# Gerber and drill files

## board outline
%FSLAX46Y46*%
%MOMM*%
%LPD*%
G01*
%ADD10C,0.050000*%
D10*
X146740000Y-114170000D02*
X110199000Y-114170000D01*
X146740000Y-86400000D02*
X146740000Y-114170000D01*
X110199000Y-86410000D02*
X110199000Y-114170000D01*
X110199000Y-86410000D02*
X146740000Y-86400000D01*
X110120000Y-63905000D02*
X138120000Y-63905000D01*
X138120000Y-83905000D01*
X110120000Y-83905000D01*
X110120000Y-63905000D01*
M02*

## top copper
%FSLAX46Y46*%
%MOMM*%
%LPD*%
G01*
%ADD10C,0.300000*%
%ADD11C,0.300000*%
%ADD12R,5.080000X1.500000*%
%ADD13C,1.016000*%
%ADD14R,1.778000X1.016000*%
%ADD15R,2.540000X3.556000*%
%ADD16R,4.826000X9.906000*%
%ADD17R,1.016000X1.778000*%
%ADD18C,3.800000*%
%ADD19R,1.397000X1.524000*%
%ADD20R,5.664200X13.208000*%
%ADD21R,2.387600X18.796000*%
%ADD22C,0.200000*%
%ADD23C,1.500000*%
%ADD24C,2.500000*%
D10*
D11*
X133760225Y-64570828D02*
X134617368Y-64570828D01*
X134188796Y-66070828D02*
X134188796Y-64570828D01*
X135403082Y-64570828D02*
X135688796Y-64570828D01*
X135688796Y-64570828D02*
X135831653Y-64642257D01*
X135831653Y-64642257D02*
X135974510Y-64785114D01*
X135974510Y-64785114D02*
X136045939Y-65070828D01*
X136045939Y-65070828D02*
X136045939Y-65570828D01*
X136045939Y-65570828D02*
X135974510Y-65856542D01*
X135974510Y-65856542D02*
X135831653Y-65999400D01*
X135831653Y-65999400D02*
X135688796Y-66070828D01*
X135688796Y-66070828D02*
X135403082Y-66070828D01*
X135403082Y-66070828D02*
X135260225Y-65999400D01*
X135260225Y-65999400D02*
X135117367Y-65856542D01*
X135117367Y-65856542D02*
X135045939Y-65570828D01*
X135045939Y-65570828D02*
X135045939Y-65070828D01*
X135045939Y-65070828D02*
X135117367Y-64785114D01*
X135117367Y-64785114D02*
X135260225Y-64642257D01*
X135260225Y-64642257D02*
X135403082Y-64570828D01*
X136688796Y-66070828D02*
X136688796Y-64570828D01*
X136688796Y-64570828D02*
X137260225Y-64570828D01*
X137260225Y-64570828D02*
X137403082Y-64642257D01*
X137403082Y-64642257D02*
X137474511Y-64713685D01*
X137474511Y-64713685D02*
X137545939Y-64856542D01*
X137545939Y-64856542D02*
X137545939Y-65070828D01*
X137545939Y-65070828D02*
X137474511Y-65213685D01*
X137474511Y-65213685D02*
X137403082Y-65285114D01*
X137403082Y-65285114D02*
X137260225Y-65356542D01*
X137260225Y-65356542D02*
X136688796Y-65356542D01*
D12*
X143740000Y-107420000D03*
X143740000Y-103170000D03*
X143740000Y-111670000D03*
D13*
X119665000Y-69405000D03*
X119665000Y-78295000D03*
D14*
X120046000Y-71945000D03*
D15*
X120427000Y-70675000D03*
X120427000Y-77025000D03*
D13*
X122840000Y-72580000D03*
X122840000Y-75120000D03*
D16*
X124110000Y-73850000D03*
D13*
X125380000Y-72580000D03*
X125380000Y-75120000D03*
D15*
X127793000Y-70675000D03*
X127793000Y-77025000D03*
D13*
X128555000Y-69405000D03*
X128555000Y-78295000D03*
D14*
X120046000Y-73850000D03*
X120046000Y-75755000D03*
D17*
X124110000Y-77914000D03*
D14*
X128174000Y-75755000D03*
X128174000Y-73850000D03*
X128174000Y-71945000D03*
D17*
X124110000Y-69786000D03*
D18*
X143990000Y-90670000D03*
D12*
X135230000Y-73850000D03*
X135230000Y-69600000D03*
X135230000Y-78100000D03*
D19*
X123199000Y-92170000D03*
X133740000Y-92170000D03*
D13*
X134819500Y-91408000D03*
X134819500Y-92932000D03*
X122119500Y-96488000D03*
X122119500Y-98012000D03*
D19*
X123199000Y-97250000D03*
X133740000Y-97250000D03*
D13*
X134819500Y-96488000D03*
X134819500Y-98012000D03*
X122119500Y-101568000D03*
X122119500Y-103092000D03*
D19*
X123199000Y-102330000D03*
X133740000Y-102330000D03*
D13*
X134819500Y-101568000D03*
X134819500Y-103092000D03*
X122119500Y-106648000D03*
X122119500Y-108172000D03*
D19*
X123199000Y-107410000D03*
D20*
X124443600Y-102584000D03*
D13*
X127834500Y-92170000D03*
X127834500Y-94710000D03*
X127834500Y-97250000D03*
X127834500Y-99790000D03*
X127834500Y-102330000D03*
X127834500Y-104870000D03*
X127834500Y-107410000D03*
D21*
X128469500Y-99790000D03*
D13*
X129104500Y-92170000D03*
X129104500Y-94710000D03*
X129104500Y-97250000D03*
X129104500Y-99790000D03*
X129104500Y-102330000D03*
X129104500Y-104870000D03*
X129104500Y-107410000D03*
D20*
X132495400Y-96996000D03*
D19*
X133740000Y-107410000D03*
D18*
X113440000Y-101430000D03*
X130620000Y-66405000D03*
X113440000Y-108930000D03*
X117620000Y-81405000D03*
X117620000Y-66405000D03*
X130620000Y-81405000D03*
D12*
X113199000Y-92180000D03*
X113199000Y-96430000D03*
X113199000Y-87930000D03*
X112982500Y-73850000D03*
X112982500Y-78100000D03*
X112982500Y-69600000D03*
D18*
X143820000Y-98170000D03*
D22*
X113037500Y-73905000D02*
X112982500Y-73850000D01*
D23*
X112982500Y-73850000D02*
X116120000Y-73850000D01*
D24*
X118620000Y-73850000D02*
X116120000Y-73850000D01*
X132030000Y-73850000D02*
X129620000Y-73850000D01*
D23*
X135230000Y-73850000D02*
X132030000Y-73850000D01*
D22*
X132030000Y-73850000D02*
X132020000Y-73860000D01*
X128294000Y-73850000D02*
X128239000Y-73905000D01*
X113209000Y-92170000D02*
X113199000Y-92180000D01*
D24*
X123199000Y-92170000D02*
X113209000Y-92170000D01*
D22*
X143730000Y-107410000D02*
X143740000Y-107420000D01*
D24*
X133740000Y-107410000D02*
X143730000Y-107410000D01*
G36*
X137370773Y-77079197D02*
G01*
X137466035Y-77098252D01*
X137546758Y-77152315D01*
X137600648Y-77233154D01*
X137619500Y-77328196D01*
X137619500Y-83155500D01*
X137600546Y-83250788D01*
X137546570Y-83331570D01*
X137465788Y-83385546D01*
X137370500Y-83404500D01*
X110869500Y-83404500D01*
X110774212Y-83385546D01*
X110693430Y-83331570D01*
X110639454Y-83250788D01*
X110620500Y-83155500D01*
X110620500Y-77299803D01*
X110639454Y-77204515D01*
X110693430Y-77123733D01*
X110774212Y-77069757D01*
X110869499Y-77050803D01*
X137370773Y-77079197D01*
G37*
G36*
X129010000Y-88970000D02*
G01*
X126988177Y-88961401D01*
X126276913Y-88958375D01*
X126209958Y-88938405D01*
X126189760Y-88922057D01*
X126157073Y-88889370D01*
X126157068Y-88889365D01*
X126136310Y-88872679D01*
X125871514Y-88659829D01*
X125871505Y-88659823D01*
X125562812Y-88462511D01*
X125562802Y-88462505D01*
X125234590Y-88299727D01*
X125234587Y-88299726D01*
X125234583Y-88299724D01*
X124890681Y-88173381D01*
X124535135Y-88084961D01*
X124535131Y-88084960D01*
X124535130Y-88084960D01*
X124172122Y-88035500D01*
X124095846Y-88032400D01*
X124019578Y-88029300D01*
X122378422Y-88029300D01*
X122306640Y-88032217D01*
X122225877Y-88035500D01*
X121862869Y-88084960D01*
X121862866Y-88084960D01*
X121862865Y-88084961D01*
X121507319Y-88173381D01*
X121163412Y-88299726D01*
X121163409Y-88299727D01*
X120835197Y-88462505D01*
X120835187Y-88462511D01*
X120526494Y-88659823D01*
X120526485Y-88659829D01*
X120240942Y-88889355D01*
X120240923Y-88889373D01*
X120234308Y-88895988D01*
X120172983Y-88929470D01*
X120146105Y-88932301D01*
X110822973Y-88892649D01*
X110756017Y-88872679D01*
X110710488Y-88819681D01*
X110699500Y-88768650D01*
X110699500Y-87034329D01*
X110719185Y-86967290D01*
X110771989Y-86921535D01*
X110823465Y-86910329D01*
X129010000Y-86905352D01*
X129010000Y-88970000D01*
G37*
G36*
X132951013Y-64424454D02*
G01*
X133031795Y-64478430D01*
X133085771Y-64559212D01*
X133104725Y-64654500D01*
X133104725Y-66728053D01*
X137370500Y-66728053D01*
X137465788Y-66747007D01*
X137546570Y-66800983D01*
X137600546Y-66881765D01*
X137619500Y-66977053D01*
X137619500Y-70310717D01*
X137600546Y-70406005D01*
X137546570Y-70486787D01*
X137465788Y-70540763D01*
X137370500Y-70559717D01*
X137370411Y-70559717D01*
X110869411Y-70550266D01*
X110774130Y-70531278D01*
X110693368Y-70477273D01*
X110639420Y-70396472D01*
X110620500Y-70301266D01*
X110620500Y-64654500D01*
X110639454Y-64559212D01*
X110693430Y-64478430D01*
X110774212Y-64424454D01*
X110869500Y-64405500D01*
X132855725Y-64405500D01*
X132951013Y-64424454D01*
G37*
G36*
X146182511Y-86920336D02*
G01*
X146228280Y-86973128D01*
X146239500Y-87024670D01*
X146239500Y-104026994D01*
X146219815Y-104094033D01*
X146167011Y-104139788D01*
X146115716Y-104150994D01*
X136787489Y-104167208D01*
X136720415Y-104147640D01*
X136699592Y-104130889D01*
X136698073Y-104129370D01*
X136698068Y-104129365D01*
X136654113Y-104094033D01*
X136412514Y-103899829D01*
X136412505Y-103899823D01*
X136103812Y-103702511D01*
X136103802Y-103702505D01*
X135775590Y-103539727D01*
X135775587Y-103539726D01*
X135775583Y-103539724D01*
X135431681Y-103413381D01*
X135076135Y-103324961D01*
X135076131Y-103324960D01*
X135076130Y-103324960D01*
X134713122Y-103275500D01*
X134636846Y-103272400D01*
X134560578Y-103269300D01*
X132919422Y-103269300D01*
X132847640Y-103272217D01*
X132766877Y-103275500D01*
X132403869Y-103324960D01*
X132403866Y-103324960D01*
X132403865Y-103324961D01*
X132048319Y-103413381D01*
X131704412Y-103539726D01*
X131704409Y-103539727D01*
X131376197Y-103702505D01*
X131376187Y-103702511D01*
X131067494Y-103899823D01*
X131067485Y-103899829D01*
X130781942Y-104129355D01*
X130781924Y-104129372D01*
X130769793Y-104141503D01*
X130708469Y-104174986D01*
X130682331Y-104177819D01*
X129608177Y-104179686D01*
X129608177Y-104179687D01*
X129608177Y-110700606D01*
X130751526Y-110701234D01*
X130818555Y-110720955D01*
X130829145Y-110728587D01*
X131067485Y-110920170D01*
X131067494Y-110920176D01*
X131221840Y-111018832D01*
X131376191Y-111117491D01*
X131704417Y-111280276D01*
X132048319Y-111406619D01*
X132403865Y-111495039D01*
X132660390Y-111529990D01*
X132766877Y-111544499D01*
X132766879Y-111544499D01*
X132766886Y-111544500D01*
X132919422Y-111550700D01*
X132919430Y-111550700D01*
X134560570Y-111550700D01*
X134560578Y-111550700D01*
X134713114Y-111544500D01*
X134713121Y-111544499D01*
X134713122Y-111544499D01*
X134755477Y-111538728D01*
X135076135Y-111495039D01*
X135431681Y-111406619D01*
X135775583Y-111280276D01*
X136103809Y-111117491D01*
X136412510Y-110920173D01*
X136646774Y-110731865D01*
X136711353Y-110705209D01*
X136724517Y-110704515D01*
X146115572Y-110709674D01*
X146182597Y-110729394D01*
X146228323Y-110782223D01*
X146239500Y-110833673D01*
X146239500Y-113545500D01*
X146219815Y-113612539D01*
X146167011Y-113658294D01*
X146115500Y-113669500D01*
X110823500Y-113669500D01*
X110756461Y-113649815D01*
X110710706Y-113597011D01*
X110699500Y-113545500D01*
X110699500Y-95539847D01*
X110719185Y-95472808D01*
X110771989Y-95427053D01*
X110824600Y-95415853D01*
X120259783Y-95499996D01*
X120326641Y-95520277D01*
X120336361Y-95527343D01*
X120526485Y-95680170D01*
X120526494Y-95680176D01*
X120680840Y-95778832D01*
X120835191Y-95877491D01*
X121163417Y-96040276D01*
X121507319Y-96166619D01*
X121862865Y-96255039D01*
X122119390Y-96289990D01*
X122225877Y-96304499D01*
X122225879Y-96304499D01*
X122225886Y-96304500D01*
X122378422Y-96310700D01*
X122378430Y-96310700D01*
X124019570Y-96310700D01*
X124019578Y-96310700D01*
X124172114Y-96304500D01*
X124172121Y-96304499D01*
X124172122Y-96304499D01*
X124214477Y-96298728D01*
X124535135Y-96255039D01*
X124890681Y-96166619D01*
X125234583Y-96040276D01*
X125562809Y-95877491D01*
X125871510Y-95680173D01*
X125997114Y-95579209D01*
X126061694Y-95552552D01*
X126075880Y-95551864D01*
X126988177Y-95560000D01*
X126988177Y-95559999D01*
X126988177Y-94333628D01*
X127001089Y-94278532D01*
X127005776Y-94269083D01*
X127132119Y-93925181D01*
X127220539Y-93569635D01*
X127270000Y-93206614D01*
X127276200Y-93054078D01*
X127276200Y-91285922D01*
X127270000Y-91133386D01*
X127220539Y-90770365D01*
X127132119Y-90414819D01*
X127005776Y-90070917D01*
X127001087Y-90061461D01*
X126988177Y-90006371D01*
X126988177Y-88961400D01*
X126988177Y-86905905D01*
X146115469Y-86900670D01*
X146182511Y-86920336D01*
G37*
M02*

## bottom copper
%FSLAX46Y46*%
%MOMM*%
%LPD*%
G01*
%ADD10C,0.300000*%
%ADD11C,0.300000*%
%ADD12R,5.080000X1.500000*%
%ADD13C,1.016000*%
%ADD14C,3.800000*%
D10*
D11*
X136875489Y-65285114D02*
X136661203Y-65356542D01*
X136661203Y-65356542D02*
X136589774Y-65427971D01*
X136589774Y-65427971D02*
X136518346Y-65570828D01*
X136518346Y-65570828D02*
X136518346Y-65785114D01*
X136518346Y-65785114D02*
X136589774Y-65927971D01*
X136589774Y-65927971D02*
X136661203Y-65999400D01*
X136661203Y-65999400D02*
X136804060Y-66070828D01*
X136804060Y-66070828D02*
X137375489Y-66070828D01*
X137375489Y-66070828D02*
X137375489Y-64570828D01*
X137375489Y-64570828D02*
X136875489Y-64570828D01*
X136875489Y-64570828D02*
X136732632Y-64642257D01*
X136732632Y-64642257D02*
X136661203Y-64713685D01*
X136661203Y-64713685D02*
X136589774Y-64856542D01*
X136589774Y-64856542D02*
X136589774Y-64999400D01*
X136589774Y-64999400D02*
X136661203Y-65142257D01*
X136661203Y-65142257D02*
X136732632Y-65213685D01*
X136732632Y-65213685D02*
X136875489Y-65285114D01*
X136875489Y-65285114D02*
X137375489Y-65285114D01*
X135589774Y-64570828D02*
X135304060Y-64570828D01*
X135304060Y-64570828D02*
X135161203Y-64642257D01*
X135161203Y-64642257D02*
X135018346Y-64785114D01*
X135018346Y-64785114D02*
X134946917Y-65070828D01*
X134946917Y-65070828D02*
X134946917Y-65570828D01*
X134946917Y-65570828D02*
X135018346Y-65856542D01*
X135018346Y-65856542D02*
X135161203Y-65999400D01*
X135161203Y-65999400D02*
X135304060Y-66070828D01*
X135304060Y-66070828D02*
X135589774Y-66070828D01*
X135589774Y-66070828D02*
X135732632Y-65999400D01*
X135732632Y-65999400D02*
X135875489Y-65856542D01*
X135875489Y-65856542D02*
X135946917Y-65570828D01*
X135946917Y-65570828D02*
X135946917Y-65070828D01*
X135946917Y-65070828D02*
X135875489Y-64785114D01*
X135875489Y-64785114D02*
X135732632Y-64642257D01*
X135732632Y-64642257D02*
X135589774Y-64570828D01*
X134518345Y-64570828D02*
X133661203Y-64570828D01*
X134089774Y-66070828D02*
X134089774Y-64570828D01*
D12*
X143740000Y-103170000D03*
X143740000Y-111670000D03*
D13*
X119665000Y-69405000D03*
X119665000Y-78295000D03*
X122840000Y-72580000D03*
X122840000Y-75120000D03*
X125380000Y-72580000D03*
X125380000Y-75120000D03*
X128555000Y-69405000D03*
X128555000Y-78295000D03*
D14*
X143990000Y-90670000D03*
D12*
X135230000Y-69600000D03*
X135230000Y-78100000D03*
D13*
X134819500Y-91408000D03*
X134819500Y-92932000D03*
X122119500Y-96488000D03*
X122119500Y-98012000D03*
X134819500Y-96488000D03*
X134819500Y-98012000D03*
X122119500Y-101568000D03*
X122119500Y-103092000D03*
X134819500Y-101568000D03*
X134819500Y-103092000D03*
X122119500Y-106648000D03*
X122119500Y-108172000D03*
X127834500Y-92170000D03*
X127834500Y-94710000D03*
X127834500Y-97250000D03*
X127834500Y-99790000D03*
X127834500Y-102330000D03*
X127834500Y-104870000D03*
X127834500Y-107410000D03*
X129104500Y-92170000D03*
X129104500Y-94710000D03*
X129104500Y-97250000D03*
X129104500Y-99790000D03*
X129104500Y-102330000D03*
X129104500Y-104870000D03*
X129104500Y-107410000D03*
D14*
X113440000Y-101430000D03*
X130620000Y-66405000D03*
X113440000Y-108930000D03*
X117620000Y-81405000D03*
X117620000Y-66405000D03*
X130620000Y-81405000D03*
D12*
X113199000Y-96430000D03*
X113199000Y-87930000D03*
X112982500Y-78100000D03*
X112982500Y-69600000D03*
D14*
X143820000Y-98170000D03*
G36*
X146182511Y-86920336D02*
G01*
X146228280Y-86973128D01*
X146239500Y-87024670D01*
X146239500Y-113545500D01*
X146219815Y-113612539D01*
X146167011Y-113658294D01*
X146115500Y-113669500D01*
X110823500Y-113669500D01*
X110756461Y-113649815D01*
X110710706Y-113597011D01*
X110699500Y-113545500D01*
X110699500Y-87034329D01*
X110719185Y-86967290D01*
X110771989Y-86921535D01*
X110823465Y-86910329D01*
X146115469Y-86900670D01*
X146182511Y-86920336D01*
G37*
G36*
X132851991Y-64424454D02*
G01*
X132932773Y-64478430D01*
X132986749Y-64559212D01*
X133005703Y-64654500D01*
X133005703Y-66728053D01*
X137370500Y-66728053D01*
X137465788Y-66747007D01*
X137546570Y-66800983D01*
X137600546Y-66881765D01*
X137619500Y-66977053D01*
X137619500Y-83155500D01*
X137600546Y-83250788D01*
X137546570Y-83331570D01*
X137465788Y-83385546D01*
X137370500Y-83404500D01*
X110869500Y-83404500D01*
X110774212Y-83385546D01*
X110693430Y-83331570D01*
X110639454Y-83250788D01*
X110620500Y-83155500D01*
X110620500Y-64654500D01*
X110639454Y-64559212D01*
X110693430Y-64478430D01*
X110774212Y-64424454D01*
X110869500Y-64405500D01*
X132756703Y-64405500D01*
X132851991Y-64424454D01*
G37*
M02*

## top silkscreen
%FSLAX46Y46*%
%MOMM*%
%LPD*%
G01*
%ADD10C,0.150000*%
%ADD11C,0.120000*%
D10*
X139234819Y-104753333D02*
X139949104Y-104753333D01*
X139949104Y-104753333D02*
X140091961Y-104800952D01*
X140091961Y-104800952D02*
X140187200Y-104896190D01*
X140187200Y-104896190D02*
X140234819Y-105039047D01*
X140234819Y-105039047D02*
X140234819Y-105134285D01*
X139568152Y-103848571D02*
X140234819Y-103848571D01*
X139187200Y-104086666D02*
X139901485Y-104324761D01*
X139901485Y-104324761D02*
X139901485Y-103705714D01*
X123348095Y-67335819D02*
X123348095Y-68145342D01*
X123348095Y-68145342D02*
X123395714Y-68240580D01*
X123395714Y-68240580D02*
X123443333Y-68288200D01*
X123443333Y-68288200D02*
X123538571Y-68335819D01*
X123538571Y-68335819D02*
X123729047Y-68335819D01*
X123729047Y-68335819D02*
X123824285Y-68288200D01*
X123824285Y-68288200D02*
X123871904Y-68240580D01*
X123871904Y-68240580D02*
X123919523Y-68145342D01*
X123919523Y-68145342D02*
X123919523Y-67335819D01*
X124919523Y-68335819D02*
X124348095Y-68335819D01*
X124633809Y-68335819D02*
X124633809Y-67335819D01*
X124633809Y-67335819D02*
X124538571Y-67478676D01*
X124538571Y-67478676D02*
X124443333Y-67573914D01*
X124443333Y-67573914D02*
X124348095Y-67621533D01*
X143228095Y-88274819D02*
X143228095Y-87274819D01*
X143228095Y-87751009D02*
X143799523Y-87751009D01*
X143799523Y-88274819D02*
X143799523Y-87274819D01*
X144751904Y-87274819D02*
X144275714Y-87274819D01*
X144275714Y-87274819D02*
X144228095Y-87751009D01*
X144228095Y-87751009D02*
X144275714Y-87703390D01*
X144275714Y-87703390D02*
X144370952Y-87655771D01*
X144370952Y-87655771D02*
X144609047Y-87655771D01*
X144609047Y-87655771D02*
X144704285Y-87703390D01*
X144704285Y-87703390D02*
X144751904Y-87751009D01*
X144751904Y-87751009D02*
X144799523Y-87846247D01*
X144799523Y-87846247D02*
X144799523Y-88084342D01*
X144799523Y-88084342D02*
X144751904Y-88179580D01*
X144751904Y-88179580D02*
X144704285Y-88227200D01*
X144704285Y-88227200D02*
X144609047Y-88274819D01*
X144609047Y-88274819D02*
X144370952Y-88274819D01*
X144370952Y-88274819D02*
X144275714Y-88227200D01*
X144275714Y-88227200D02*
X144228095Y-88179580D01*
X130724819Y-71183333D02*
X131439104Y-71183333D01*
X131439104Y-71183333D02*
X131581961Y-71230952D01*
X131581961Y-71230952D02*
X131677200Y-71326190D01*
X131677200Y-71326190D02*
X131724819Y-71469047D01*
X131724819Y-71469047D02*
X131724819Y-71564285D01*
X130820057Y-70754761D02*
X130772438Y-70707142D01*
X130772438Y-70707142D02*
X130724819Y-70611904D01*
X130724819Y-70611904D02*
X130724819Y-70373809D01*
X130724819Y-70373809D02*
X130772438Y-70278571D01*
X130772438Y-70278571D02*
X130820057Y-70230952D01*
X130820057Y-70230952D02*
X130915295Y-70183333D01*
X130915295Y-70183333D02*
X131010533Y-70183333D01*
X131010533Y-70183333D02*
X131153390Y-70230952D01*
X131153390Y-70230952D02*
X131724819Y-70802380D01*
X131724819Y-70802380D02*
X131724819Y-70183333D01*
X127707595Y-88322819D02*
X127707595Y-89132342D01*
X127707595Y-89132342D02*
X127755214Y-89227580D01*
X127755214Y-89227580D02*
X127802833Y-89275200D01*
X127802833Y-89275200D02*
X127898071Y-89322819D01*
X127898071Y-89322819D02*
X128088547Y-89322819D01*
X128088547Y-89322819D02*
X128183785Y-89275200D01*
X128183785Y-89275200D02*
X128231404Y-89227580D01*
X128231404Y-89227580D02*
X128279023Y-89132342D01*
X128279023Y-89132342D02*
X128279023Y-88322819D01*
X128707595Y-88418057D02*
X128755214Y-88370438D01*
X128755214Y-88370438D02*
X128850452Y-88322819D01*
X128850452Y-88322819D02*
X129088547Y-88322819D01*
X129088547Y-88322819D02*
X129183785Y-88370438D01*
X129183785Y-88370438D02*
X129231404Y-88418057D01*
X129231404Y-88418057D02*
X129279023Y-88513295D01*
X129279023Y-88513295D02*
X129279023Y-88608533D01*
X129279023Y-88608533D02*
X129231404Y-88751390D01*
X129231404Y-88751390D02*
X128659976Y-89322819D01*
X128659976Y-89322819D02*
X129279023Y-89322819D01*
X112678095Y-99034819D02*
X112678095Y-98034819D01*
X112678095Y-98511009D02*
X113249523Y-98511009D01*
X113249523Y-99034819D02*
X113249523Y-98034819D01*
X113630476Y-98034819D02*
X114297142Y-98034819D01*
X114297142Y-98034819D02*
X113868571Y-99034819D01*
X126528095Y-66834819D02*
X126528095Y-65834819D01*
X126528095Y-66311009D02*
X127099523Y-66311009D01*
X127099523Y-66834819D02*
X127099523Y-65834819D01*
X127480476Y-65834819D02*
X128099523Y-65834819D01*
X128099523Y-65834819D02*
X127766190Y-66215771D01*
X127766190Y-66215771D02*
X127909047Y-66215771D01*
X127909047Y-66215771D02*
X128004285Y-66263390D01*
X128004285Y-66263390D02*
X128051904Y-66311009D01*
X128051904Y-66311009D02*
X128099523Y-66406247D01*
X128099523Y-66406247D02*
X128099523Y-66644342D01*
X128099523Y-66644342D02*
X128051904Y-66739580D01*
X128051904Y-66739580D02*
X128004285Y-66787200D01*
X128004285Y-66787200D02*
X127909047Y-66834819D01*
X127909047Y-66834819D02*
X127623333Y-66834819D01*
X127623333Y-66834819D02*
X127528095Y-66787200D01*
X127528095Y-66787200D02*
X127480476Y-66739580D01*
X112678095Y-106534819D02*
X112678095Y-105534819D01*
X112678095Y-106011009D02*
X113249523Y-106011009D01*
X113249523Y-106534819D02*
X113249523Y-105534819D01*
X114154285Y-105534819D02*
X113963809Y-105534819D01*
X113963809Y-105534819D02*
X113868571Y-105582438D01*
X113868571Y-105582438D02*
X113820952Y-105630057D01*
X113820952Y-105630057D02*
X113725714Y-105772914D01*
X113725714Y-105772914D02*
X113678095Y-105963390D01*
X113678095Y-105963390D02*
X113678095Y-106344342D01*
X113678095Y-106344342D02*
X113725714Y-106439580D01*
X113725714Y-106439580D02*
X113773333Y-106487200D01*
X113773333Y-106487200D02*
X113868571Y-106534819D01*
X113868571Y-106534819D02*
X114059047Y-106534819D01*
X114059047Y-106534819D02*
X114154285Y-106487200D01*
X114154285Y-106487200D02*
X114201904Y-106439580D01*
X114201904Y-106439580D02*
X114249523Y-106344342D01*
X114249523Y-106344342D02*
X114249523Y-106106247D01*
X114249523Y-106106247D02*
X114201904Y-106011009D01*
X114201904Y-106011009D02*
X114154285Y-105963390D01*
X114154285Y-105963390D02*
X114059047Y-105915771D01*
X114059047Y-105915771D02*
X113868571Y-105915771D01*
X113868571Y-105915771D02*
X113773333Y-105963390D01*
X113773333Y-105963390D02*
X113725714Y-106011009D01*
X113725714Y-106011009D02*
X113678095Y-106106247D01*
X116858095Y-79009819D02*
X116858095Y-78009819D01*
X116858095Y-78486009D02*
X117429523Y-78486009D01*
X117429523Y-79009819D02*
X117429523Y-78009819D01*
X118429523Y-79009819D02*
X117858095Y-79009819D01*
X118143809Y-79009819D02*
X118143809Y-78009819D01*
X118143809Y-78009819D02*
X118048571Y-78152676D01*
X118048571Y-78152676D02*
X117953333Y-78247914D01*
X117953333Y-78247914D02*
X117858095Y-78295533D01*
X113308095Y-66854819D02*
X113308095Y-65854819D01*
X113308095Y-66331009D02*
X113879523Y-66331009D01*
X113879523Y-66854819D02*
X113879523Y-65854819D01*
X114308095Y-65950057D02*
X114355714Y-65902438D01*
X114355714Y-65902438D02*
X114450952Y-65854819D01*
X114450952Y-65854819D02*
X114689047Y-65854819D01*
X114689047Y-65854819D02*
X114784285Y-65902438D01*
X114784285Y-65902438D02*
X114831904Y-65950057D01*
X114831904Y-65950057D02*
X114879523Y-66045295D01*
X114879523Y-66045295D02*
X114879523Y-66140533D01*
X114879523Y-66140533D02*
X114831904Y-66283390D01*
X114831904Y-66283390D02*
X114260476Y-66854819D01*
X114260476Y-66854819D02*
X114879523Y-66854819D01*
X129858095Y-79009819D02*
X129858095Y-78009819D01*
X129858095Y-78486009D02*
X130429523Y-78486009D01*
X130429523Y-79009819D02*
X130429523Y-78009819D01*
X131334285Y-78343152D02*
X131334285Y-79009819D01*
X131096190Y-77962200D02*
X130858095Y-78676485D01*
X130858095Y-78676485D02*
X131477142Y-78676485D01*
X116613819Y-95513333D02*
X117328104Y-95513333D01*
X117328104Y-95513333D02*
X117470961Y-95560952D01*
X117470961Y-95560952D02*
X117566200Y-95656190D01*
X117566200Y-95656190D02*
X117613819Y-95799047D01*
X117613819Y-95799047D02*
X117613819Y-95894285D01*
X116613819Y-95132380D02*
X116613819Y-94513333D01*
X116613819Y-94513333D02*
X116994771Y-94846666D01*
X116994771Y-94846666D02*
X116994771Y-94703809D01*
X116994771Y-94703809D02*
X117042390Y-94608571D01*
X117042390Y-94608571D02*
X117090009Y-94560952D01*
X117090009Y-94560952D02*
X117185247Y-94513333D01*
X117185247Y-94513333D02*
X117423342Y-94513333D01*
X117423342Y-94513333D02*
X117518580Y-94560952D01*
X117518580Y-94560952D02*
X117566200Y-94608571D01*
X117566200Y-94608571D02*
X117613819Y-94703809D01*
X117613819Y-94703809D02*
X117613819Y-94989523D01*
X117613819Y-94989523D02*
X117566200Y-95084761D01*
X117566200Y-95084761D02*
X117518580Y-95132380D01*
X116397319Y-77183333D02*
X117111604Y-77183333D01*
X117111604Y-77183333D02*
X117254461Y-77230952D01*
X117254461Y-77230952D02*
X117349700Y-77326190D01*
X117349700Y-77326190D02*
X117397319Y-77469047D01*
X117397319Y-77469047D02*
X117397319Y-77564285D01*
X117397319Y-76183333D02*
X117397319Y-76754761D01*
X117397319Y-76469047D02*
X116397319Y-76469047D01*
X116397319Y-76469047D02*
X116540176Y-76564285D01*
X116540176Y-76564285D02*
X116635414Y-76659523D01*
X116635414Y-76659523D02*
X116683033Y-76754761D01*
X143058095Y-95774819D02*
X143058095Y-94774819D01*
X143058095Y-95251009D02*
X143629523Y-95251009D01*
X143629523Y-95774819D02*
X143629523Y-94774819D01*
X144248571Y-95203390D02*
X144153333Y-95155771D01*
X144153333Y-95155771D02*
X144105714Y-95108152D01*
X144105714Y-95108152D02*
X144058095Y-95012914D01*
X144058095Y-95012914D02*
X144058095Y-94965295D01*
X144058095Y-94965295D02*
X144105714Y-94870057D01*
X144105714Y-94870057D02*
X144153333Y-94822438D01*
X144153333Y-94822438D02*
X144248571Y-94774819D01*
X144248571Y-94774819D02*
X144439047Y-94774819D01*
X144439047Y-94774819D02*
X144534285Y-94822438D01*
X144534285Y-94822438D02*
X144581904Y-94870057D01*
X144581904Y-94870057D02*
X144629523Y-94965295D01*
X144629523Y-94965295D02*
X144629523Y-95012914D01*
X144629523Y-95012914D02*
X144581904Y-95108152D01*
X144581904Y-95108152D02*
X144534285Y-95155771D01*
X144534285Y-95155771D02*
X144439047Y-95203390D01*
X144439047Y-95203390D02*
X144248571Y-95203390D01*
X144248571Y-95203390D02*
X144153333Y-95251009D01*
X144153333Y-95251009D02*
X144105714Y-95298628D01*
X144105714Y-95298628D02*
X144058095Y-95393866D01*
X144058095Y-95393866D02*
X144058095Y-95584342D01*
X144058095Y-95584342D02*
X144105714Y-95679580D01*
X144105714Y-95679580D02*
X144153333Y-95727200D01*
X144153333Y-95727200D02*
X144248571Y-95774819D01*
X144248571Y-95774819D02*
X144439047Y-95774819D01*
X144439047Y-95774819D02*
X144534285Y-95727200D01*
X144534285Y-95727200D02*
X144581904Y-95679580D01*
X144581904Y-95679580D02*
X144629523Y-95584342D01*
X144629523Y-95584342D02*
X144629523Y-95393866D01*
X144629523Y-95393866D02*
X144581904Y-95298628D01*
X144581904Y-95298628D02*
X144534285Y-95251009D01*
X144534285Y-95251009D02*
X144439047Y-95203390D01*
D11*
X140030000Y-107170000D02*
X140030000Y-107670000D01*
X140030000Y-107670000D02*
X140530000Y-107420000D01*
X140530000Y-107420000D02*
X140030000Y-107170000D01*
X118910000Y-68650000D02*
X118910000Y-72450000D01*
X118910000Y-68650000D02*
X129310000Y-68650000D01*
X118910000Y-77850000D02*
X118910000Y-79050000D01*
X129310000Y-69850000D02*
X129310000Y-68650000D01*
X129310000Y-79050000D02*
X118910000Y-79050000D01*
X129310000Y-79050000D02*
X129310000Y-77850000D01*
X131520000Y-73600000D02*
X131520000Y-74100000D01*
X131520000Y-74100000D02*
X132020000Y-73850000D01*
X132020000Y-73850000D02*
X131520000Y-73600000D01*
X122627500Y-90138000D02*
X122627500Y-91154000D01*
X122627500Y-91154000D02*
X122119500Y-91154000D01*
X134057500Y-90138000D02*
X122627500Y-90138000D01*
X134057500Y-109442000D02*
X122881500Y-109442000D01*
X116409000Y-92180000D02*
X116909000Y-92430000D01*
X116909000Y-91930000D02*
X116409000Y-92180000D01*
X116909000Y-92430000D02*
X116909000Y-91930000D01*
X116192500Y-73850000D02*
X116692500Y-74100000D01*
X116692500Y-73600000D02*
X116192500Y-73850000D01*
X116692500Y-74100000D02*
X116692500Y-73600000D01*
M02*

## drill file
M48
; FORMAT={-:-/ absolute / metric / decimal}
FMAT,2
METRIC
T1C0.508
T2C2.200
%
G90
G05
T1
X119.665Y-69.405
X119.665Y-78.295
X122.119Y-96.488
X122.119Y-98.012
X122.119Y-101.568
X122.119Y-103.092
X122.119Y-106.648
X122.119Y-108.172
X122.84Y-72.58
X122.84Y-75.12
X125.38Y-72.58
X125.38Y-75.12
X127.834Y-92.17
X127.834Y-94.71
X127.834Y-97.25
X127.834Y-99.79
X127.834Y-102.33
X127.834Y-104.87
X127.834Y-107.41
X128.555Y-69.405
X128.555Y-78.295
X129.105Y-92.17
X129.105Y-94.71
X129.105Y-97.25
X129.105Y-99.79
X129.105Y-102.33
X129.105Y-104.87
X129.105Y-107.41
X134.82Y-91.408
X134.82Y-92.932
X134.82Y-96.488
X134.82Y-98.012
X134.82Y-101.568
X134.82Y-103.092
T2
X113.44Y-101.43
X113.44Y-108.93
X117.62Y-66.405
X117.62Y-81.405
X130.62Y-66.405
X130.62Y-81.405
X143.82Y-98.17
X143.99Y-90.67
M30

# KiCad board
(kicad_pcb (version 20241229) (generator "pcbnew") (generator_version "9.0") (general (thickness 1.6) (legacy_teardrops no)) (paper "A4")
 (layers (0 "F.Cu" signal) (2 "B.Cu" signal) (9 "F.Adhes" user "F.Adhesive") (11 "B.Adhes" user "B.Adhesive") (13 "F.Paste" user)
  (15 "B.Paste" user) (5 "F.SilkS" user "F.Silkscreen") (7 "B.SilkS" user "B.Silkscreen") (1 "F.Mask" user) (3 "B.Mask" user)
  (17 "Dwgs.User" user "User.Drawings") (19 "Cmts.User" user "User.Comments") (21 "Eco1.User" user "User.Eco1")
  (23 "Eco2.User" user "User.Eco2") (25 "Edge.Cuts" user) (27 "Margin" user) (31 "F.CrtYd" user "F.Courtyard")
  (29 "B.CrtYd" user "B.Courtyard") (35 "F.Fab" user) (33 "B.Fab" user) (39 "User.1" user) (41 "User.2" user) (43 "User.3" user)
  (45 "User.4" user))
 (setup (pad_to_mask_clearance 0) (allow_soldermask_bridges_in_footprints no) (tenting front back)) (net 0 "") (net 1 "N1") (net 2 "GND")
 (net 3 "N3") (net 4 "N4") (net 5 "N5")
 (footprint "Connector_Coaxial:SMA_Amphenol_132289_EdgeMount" (layer "F.Cu") (at 143.74 107.42)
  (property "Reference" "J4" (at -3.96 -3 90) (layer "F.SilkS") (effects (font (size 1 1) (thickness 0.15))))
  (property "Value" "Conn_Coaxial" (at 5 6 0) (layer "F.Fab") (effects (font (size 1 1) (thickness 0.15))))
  (fp_line (start -3.71 -0.25) (end -3.71 0.25) (stroke (width 0.12) (type solid)) (layer "F.SilkS"))
  (fp_line (start -3.71 0.25) (end -3.21 0) (stroke (width 0.12) (type solid)) (layer "F.SilkS"))
  (fp_line (start -3.21 0) (end -3.71 -0.25) (stroke (width 0.12) (type solid)) (layer "F.SilkS"))
  (pad "1" smd rect (at 0 0 90) (size 1.5 5.08) (layers "F.Cu" "F.Mask" "F.Paste") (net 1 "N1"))
  (pad "2" smd rect (at 0 -4.25 90) (size 1.5 5.08) (layers "F.Cu" "F.Mask" "F.Paste") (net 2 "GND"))
  (pad "2" smd rect (at 0 -4.25 90) (size 1.5 5.08) (layers "B.Cu" "B.Mask" "B.Paste") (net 2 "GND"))
  (pad "2" smd rect (at 0 4.25 90) (size 1.5 5.08) (layers "F.Cu" "F.Mask" "F.Paste") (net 2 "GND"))
  (pad "2" smd rect (at 0 4.25 90) (size 1.5 5.08) (layers "B.Cu" "B.Mask" "B.Paste") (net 2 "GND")))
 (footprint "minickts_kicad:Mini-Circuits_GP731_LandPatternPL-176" (layer "F.Cu") (at 124.11 73.85)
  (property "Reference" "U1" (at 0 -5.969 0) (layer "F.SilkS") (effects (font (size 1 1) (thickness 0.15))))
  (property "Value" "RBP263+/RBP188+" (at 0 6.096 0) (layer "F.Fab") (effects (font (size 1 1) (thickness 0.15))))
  (fp_line (start -5.2 -5.2) (end -5.2 -1.4) (stroke (width 0.12) (type solid)) (layer "F.SilkS"))
  (fp_line (start -5.2 -5.2) (end 5.2 -5.2) (stroke (width 0.12) (type solid)) (layer "F.SilkS"))
  (fp_line (start -5.2 4) (end -5.2 5.2) (stroke (width 0.12) (type solid)) (layer "F.SilkS"))
  (fp_line (start 5.2 -4) (end 5.2 -5.2) (stroke (width 0.12) (type solid)) (layer "F.SilkS"))
  (fp_line (start 5.2 5.2) (end -5.2 5.2) (stroke (width 0.12) (type solid)) (layer "F.SilkS"))
  (fp_line (start 5.2 5.2) (end 5.2 4) (stroke (width 0.12) (type solid)) (layer "F.SilkS"))
  (pad "1" thru_hole circle (at -4.445 -4.445) (size 1.016 1.016) (drill 0.508) (layers "*.Cu") (remove_unused_layers no) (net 2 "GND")
   (zone_connect 2))
  (pad "1" thru_hole circle (at -4.445 4.445) (size 1.016 1.016) (drill 0.508) (layers "*.Cu") (remove_unused_layers no) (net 2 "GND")
   (zone_connect 2))
  (pad "1" smd rect (at -4.064 -1.905 180) (size 1.778 1.016) (layers "F.Cu" "F.Mask" "F.Paste") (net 2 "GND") (zone_connect 2))
  (pad "1" smd rect (at -3.683 -3.175) (size 2.54 3.556) (layers "F.Cu") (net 2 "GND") (zone_connect 2))
  (pad "1" smd rect (at -3.683 3.175) (size 2.54 3.556) (layers "F.Cu") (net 2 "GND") (zone_connect 2))
  (pad "1" thru_hole circle (at -1.27 -1.27) (size 1.016 1.016) (drill 0.508) (layers "*.Cu") (remove_unused_layers no) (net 2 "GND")
   (zone_connect 2))
  (pad "1" thru_hole circle (at -1.27 1.27) (size 1.016 1.016) (drill 0.508) (layers "*.Cu") (remove_unused_layers no) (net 2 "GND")
   (zone_connect 2))
  (pad "1" smd rect (at 0 0) (size 4.826 9.906) (layers "F.Cu") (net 2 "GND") (zone_connect 2))
  (pad "1" thru_hole circle (at 1.27 -1.27) (size 1.016 1.016) (drill 0.508) (layers "*.Cu") (remove_unused_layers no) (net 2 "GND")
   (zone_connect 2))
  (pad "1" thru_hole circle (at 1.27 1.27) (size 1.016 1.016) (drill 0.508) (layers "*.Cu") (remove_unused_layers no) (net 2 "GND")
   (zone_connect 2))
  (pad "1" smd rect (at 3.683 -3.175) (size 2.54 3.556) (layers "F.Cu") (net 2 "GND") (zone_connect 2))
  (pad "1" smd rect (at 3.683 3.175) (size 2.54 3.556) (layers "F.Cu") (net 2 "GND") (zone_connect 2))
  (pad "1" thru_hole circle (at 4.445 -4.445) (size 1.016 1.016) (drill 0.508) (layers "*.Cu") (remove_unused_layers no) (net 2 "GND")
   (zone_connect 2))
  (pad "1" thru_hole circle (at 4.445 4.445) (size 1.016 1.016) (drill 0.508) (layers "*.Cu") (remove_unused_layers no) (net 2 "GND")
   (zone_connect 2))
  (pad "2" smd rect (at -4.064 0 180) (size 1.778 1.016) (layers "F.Cu" "F.Mask" "F.Paste") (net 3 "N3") (clearance 0.762))
  (pad "3" smd rect (at -4.064 1.905 180) (size 1.778 1.016) (layers "F.Cu" "F.Mask" "F.Paste") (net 2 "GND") (zone_connect 2))
  (pad "4" smd rect (at 0 4.064 270) (size 1.778 1.016) (layers "F.Cu" "F.Mask" "F.Paste") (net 2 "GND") (zone_connect 2))
  (pad "5" smd rect (at 4.064 1.905) (size 1.778 1.016) (layers "F.Cu" "F.Mask" "F.Paste") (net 2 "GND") (zone_connect 2))
  (pad "6" smd rect (at 4.064 0) (size 1.778 1.016) (layers "F.Cu" "F.Mask" "F.Paste") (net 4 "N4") (clearance 0.762))
  (pad "7" smd rect (at 4.064 -1.905) (size 1.778 1.016) (layers "F.Cu" "F.Mask" "F.Paste") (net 2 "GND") (zone_connect 2))
  (pad "8" smd rect (at 0 -4.064 270) (size 1.778 1.016) (layers "F.Cu" "F.Mask" "F.Paste") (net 2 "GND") (zone_connect 2)))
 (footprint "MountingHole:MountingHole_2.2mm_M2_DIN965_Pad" (layer "F.Cu") (at 143.99 90.67)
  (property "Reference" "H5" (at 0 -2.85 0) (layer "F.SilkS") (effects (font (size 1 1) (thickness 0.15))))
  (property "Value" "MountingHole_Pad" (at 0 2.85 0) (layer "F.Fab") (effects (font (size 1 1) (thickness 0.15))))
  (pad "1" thru_hole circle (at 0 0) (size 3.8 3.8) (drill 2.2) (layers "*.Cu" "*.Mask") (remove_unused_layers no) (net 2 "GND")
   (zone_connect 2)))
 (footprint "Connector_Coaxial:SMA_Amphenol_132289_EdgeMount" (layer "F.Cu") (at 135.23 73.85)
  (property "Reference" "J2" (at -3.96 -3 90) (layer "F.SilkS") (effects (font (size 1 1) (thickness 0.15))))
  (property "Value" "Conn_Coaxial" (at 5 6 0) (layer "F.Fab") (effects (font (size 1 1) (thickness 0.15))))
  (fp_line (start -3.71 -0.25) (end -3.71 0.25) (stroke (width 0.12) (type solid)) (layer "F.SilkS"))
  (fp_line (start -3.71 0.25) (end -3.21 0) (stroke (width 0.12) (type solid)) (layer "F.SilkS"))
  (fp_line (start -3.21 0) (end -3.71 -0.25) (stroke (width 0.12) (type solid)) (layer "F.SilkS"))
  (pad "1" smd rect (at 0 0 90) (size 1.5 5.08) (layers "F.Cu" "F.Mask" "F.Paste") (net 4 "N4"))
  (pad "2" smd rect (at 0 -4.25 90) (size 1.5 5.08) (layers "F.Cu" "F.Mask" "F.Paste") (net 2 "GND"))
  (pad "2" smd rect (at 0 -4.25 90) (size 1.5 5.08) (layers "B.Cu" "B.Mask" "B.Paste") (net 2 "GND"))
  (pad "2" smd rect (at 0 4.25 90) (size 1.5 5.08) (layers "F.Cu" "F.Mask" "F.Paste") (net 2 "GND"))
  (pad "2" smd rect (at 0 4.25 90) (size 1.5 5.08) (layers "B.Cu" "B.Mask" "B.Paste") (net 2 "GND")))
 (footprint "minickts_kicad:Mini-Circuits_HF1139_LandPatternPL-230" (layer "F.Cu") (at 128.4695 99.79)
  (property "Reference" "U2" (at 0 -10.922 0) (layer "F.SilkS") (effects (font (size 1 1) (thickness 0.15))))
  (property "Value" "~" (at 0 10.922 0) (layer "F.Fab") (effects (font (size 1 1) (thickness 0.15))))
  (fp_line (start -5.842 -9.652) (end -5.842 -8.636) (stroke (width 0.12) (type solid)) (layer "F.SilkS"))
  (fp_line (start -5.842 -8.636) (end -6.35 -8.636) (stroke (width 0.12) (type solid)) (layer "F.SilkS"))
  (fp_line (start 5.588 -9.652) (end -5.842 -9.652) (stroke (width 0.12) (type solid)) (layer "F.SilkS"))
  (fp_line (start 5.588 9.652) (end -5.588 9.652) (stroke (width 0.12) (type solid)) (layer "F.SilkS"))
  (pad "1" smd rect (at -5.2705 -7.62 270) (size 1.524 1.397) (layers "F.Cu" "F.Mask" "F.Paste") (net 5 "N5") (clearance 3.3782))
  (pad "2" smd rect (at 5.2705 -7.62 270) (size 1.524 1.397) (layers "F.Cu" "F.Mask" "F.Paste") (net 2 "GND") (zone_connect 2))
  (pad "2" thru_hole circle (at 6.35 -8.382 270) (size 1.016 1.016) (drill 0.508) (layers "*.Cu") (remove_unused_layers no) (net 2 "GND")
   (zone_connect 2))
  (pad "2" thru_hole circle (at 6.35 -6.858 270) (size 1.016 1.016) (drill 0.508) (layers "*.Cu") (remove_unused_layers no) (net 2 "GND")
   (zone_connect 2))
  (pad "3" thru_hole circle (at -6.35 -3.302 270) (size 1.016 1.016) (drill 0.508) (layers "*.Cu") (remove_unused_layers no) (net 2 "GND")
   (zone_connect 2))
  (pad "3" thru_hole circle (at -6.35 -1.778 270) (size 1.016 1.016) (drill 0.508) (layers "*.Cu") (remove_unused_layers no) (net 2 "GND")
   (zone_connect 2))
  (pad "3" smd rect (at -5.2705 -2.54 270) (size 1.524 1.397) (layers "F.Cu" "F.Mask" "F.Paste") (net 2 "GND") (zone_connect 2))
  (pad "4" smd rect (at 5.2705 -2.54 270) (size 1.524 1.397) (layers "F.Cu" "F.Mask" "F.Paste") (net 2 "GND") (zone_connect 2))
  (pad "4" thru_hole circle (at 6.35 -3.302 270) (size 1.016 1.016) (drill 0.508) (layers "*.Cu") (remove_unused_layers no) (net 2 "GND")
   (zone_connect 2))
  (pad "4" thru_hole circle (at 6.35 -1.778 270) (size 1.016 1.016) (drill 0.508) (layers "*.Cu") (remove_unused_layers no) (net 2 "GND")
   (zone_connect 2))
  (pad "5" thru_hole circle (at -6.35 1.778 270) (size 1.016 1.016) (drill 0.508) (layers "*.Cu") (remove_unused_layers no) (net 2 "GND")
   (zone_connect 2))
  (pad "5" thru_hole circle (at -6.35 3.302 270) (size 1.016 1.016) (drill 0.508) (layers "*.Cu") (remove_unused_layers no) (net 2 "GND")
   (zone_connect 2))
  (pad "5" smd rect (at -5.2705 2.54 270) (size 1.524 1.397) (layers "F.Cu" "F.Mask" "F.Paste") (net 2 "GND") (zone_connect 2))
  (pad "6" smd rect (at 5.2705 2.54 270) (size 1.524 1.397) (layers "F.Cu" "F.Mask" "F.Paste") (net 2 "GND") (zone_connect 2))
  (pad "6" thru_hole circle (at 6.35 1.778 270) (size 1.016 1.016) (drill 0.508) (layers "*.Cu") (remove_unused_layers no) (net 2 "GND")
   (zone_connect 2))
  (pad "6" thru_hole circle (at 6.35 3.302 270) (size 1.016 1.016) (drill 0.508) (layers "*.Cu") (remove_unused_layers no) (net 2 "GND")
   (zone_connect 2))
  (pad "7" thru_hole circle (at -6.35 6.858 270) (size 1.016 1.016) (drill 0.508) (layers "*.Cu") (remove_unused_layers no) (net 2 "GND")
   (zone_connect 2))
  (pad "7" thru_hole circle (at -6.35 8.382 270) (size 1.016 1.016) (drill 0.508) (layers "*.Cu") (remove_unused_layers no) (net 2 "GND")
   (zone_connect 2))
  (pad "7" smd rect (at -5.2705 7.62 270) (size 1.524 1.397) (layers "F.Cu" "F.Mask" "F.Paste") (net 2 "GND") (zone_connect 2))
  (pad "7" smd rect (at -4.0259 2.794 270) (size 13.208 5.6642) (layers "F.Cu") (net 2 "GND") (zone_connect 2))
  (pad "7" thru_hole circle (at -0.635 -7.62 270) (size 1.016 1.016) (drill 0.508) (layers "*.Cu") (remove_unused_layers no) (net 2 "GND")
   (zone_connect 2))
  (pad "7" thru_hole circle (at -0.635 -5.08 270) (size 1.016 1.016) (drill 0.508) (layers "*.Cu") (remove_unused_layers no) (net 2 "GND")
   (zone_connect 2))
  (pad "7" thru_hole circle (at -0.635 -2.54 270) (size 1.016 1.016) (drill 0.508) (layers "*.Cu") (remove_unused_layers no) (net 2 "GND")
   (zone_connect 2))
  (pad "7" thru_hole circle (at -0.635 0 270) (size 1.016 1.016) (drill 0.508) (layers "*.Cu") (remove_unused_layers no) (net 2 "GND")
   (zone_connect 2))
  (pad "7" thru_hole circle (at -0.635 2.54 270) (size 1.016 1.016) (drill 0.508) (layers "*.Cu") (remove_unused_layers no) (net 2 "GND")
   (zone_connect 2))
  (pad "7" thru_hole circle (at -0.635 5.08 270) (size 1.016 1.016) (drill 0.508) (layers "*.Cu") (remove_unused_layers no) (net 2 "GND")
   (zone_connect 2))
  (pad "7" thru_hole circle (at -0.635 7.62 270) (size 1.016 1.016) (drill 0.508) (layers "*.Cu") (remove_unused_layers no) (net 2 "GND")
   (zone_connect 2))
  (pad "7" smd rect (at 0 0 270) (size 18.796 2.3876) (layers "F.Cu") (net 2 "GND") (zone_connect 2))
  (pad "7" thru_hole circle (at 0.635 -7.62 270) (size 1.016 1.016) (drill 0.508) (layers "*.Cu") (remove_unused_layers no) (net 2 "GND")
   (zone_connect 2))
  (pad "7" thru_hole circle (at 0.635 -5.08 270) (size 1.016 1.016) (drill 0.508) (layers "*.Cu") (remove_unused_layers no) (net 2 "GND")
   (zone_connect 2))
  (pad "7" thru_hole circle (at 0.635 -2.54 270) (size 1.016 1.016) (drill 0.508) (layers "*.Cu") (remove_unused_layers no) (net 2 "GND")
   (zone_connect 2))
  (pad "7" thru_hole circle (at 0.635 0 270) (size 1.016 1.016) (drill 0.508) (layers "*.Cu") (remove_unused_layers no) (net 2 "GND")
   (zone_connect 2))
  (pad "7" thru_hole circle (at 0.635 2.54 270) (size 1.016 1.016) (drill 0.508) (layers "*.Cu") (remove_unused_layers no) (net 2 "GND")
   (zone_connect 2))
  (pad "7" thru_hole circle (at 0.635 5.08 270) (size 1.016 1.016) (drill 0.508) (layers "*.Cu") (remove_unused_layers no) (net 2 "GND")
   (zone_connect 2))
  (pad "7" thru_hole circle (at 0.635 7.62 270) (size 1.016 1.016) (drill 0.508) (layers "*.Cu") (remove_unused_layers no) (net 2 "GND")
   (zone_connect 2))
  (pad "7" smd rect (at 4.0259 -2.794 270) (size 13.208 5.6642) (layers "F.Cu") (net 2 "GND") (zone_connect 2))
  (pad "8" smd rect (at 5.2705 7.62 270) (size 1.524 1.397) (layers "F.Cu" "F.Mask" "F.Paste") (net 1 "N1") (clearance 3.3782)))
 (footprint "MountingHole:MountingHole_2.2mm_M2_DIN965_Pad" (layer "F.Cu") (at 113.44 101.43)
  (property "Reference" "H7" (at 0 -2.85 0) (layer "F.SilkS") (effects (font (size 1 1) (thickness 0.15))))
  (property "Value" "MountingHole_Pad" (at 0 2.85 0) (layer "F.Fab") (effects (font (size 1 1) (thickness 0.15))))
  (pad "1" thru_hole circle (at 0 0) (size 3.8 3.8) (drill 2.2) (layers "*.Cu" "*.Mask") (remove_unused_layers no) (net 2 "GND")
   (zone_connect 2)))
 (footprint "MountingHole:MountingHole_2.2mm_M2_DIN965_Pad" (layer "F.Cu") (at 130.62 66.405)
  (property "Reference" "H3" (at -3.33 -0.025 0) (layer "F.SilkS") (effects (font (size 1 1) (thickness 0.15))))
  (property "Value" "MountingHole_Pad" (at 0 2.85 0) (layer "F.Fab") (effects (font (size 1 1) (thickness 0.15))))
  (pad "1" thru_hole circle (at 0 0) (size 3.8 3.8) (drill 2.2) (layers "*.Cu" "*.Mask") (remove_unused_layers no) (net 2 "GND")
   (zone_connect 2)))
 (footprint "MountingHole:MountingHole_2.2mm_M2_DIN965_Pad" (layer "F.Cu") (at 113.44 108.93)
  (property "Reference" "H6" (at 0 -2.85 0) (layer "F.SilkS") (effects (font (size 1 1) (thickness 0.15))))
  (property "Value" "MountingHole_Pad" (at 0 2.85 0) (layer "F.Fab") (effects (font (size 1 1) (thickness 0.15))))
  (pad "1" thru_hole circle (at 0 0) (size 3.8 3.8) (drill 2.2) (layers "*.Cu" "*.Mask") (remove_unused_layers no) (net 2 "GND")
   (zone_connect 2)))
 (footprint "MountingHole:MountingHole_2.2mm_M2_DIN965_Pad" (layer "F.Cu") (at 117.62 81.405)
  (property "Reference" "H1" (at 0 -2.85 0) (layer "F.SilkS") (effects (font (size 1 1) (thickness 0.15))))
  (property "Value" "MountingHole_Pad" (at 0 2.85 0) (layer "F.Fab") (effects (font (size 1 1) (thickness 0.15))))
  (pad "1" thru_hole circle (at 0 0) (size 3.8 3.8) (drill 2.2) (layers "*.Cu" "*.Mask") (remove_unused_layers no) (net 2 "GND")
   (zone_connect 2)))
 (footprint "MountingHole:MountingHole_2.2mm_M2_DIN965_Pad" (layer "F.Cu") (at 117.62 66.405)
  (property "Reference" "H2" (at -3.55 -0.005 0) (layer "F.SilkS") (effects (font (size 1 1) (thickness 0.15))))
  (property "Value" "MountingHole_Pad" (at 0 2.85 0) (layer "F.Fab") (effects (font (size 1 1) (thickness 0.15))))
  (pad "1" thru_hole circle (at 0 0) (size 3.8 3.8) (drill 2.2) (layers "*.Cu" "*.Mask") (remove_unused_layers no) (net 2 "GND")
   (zone_connect 2)))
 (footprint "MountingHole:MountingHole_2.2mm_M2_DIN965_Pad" (layer "F.Cu") (at 130.62 81.405)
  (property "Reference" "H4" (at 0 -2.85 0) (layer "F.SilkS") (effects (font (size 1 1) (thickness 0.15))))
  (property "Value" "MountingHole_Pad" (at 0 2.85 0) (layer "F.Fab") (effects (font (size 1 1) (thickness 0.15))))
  (pad "1" thru_hole circle (at 0 0) (size 3.8 3.8) (drill 2.2) (layers "*.Cu" "*.Mask") (remove_unused_layers no) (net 2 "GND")
   (zone_connect 2)))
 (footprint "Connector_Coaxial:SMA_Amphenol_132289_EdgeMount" (layer "F.Cu") (at 113.199 92.18 180)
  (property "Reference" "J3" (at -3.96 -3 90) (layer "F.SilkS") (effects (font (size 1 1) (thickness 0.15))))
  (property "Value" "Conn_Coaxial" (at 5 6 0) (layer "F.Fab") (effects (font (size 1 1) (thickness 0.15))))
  (fp_line (start -3.21 0) (end -3.71 -0.25) (stroke (width 0.12) (type solid)) (layer "F.SilkS"))
  (fp_line (start -3.71 0.25) (end -3.21 0) (stroke (width 0.12) (type solid)) (layer "F.SilkS"))
  (fp_line (start -3.71 -0.25) (end -3.71 0.25) (stroke (width 0.12) (type solid)) (layer "F.SilkS"))
  (pad "1" smd rect (at 0 0 270) (size 1.5 5.08) (layers "F.Cu" "F.Mask" "F.Paste") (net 5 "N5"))
  (pad "2" smd rect (at 0 -4.25 270) (size 1.5 5.08) (layers "F.Cu" "F.Mask" "F.Paste") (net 2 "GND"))
  (pad "2" smd rect (at 0 -4.25 270) (size 1.5 5.08) (layers "B.Cu" "B.Mask" "B.Paste") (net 2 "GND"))
  (pad "2" smd rect (at 0 4.25 270) (size 1.5 5.08) (layers "F.Cu" "F.Mask" "F.Paste") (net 2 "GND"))
  (pad "2" smd rect (at 0 4.25 270) (size 1.5 5.08) (layers "B.Cu" "B.Mask" "B.Paste") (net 2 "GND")))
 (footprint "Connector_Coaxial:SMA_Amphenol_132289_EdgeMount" (layer "F.Cu") (at 112.9825 73.85 180)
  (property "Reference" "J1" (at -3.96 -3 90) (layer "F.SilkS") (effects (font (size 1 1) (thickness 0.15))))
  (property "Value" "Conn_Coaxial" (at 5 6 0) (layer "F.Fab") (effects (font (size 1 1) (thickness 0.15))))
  (fp_line (start -3.21 0) (end -3.71 -0.25) (stroke (width 0.12) (type solid)) (layer "F.SilkS"))
  (fp_line (start -3.71 0.25) (end -3.21 0) (stroke (width 0.12) (type solid)) (layer "F.SilkS"))
  (fp_line (start -3.71 -0.25) (end -3.71 0.25) (stroke (width 0.12) (type solid)) (layer "F.SilkS"))
  (pad "1" smd rect (at 0 0 270) (size 1.5 5.08) (layers "F.Cu" "F.Mask" "F.Paste") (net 3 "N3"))
  (pad "2" smd rect (at 0 -4.25 270) (size 1.5 5.08) (layers "F.Cu" "F.Mask" "F.Paste") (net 2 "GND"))
  (pad "2" smd rect (at 0 -4.25 270) (size 1.5 5.08) (layers "B.Cu" "B.Mask" "B.Paste") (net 2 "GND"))
  (pad "2" smd rect (at 0 4.25 270) (size 1.5 5.08) (layers "F.Cu" "F.Mask" "F.Paste") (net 2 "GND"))
  (pad "2" smd rect (at 0 4.25 270) (size 1.5 5.08) (layers "B.Cu" "B.Mask" "B.Paste") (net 2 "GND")))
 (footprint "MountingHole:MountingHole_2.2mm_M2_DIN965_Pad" (layer "F.Cu") (at 143.82 98.17)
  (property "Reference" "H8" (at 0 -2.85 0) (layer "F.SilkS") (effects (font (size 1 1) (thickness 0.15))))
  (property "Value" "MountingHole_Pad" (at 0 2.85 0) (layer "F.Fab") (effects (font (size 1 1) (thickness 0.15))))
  (pad "1" thru_hole circle (at 0 0) (size 3.8 3.8) (drill 2.2) (layers "*.Cu" "*.Mask") (remove_unused_layers no) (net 2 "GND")
   (zone_connect 2)))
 (gr_line (start 146.74 114.17) (end 110.199 114.17) (stroke (width 0.05) (type solid)) (layer "Edge.Cuts"))
 (gr_line (start 146.74 86.4) (end 146.74 114.17) (stroke (width 0.05) (type solid)) (layer "Edge.Cuts"))
 (gr_line (start 110.199 86.41) (end 110.199 114.17) (stroke (width 0.05) (type default)) (layer "Edge.Cuts"))
 (gr_line (start 110.199 86.41) (end 146.74 86.4) (stroke (width 0.05) (type solid)) (layer "Edge.Cuts"))
 (gr_rect (start 110.12 63.905) (end 138.12 83.905) (stroke (width 0.05) (type solid)) (fill no) (layer "Edge.Cuts"))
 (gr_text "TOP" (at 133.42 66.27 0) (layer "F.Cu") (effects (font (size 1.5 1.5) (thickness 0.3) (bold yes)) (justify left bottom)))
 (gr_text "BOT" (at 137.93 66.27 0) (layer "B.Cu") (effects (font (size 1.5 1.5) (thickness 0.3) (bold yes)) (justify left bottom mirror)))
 (segment (start 113.0375 73.905) (end 112.9825 73.85) (width 0.2) (layer "F.Cu") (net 3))
 (segment (start 112.9825 73.85) (end 116.12 73.85) (width 1.5) (layer "F.Cu") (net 3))
 (segment (start 118.62 73.85) (end 116.12 73.85) (width 2.5) (layer "F.Cu") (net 3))
 (segment (start 132.03 73.85) (end 129.62 73.85) (width 2.5) (layer "F.Cu") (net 4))
 (segment (start 135.23 73.85) (end 132.03 73.85) (width 1.5) (layer "F.Cu") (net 4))
 (segment (start 132.03 73.85) (end 132.02 73.86) (width 0.2) (layer "F.Cu") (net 4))
 (segment (start 128.294 73.85) (end 128.239 73.905) (width 0.2) (layer "F.Cu") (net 4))
 (segment (start 113.209 92.17) (end 113.199 92.18) (width 0.2) (layer "F.Cu") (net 5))
 (segment (start 123.199 92.17) (end 113.209 92.17) (width 2.5) (layer "F.Cu") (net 5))
 (segment (start 143.73 107.41) (end 143.74 107.42) (width 0.2) (layer "F.Cu") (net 1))
 (segment (start 133.74 107.41) (end 143.73 107.41) (width 2.5) (layer "F.Cu") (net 1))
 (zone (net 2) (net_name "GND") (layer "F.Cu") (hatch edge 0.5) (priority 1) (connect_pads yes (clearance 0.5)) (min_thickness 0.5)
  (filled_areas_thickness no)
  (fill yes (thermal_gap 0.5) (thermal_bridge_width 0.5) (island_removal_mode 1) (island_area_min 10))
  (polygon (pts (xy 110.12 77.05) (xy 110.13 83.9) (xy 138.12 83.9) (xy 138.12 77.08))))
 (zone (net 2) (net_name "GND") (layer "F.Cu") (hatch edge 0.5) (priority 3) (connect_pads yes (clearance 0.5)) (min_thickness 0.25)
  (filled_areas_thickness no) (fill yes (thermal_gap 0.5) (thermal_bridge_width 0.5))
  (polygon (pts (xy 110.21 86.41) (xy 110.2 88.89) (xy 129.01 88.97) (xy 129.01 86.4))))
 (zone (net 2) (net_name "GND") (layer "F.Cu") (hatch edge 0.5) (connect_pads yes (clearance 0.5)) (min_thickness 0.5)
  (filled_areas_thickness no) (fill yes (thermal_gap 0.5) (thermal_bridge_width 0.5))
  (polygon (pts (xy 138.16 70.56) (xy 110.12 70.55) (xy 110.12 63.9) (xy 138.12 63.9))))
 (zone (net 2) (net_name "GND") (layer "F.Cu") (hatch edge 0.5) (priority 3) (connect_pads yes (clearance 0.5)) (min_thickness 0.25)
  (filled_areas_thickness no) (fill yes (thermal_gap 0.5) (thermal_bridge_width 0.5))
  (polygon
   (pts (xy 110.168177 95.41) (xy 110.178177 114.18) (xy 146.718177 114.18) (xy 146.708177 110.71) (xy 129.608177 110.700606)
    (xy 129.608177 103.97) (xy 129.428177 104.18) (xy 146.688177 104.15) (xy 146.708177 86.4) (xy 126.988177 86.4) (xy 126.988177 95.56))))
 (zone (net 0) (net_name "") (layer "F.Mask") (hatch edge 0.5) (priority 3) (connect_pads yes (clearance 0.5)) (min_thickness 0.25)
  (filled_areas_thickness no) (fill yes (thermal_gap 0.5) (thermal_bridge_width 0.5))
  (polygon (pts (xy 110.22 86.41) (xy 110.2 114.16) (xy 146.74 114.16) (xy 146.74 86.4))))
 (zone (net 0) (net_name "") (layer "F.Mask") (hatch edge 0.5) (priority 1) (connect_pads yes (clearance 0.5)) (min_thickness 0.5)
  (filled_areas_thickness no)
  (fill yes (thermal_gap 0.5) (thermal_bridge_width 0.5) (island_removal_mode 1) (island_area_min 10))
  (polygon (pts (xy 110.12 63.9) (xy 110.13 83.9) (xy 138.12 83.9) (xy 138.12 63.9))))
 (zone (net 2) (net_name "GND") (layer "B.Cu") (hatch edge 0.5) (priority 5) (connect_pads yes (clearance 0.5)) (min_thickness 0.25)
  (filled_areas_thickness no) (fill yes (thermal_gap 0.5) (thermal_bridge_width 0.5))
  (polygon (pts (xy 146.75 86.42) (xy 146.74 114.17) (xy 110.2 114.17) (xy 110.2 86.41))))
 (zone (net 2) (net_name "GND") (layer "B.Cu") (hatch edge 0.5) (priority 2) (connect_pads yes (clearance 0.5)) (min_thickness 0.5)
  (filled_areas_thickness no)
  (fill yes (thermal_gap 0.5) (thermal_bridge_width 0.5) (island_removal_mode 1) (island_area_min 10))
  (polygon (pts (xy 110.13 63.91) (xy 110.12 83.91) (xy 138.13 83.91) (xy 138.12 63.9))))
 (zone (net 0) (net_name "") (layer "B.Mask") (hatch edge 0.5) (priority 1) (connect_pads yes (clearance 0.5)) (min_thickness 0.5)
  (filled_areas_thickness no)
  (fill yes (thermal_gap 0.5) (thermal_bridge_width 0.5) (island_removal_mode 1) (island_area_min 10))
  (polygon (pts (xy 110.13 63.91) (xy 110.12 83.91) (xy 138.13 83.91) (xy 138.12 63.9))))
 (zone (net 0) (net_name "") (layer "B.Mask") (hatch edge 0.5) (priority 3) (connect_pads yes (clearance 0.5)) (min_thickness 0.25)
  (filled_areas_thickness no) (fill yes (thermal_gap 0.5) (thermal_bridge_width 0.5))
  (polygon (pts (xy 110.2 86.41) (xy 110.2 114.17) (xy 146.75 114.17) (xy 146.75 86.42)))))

